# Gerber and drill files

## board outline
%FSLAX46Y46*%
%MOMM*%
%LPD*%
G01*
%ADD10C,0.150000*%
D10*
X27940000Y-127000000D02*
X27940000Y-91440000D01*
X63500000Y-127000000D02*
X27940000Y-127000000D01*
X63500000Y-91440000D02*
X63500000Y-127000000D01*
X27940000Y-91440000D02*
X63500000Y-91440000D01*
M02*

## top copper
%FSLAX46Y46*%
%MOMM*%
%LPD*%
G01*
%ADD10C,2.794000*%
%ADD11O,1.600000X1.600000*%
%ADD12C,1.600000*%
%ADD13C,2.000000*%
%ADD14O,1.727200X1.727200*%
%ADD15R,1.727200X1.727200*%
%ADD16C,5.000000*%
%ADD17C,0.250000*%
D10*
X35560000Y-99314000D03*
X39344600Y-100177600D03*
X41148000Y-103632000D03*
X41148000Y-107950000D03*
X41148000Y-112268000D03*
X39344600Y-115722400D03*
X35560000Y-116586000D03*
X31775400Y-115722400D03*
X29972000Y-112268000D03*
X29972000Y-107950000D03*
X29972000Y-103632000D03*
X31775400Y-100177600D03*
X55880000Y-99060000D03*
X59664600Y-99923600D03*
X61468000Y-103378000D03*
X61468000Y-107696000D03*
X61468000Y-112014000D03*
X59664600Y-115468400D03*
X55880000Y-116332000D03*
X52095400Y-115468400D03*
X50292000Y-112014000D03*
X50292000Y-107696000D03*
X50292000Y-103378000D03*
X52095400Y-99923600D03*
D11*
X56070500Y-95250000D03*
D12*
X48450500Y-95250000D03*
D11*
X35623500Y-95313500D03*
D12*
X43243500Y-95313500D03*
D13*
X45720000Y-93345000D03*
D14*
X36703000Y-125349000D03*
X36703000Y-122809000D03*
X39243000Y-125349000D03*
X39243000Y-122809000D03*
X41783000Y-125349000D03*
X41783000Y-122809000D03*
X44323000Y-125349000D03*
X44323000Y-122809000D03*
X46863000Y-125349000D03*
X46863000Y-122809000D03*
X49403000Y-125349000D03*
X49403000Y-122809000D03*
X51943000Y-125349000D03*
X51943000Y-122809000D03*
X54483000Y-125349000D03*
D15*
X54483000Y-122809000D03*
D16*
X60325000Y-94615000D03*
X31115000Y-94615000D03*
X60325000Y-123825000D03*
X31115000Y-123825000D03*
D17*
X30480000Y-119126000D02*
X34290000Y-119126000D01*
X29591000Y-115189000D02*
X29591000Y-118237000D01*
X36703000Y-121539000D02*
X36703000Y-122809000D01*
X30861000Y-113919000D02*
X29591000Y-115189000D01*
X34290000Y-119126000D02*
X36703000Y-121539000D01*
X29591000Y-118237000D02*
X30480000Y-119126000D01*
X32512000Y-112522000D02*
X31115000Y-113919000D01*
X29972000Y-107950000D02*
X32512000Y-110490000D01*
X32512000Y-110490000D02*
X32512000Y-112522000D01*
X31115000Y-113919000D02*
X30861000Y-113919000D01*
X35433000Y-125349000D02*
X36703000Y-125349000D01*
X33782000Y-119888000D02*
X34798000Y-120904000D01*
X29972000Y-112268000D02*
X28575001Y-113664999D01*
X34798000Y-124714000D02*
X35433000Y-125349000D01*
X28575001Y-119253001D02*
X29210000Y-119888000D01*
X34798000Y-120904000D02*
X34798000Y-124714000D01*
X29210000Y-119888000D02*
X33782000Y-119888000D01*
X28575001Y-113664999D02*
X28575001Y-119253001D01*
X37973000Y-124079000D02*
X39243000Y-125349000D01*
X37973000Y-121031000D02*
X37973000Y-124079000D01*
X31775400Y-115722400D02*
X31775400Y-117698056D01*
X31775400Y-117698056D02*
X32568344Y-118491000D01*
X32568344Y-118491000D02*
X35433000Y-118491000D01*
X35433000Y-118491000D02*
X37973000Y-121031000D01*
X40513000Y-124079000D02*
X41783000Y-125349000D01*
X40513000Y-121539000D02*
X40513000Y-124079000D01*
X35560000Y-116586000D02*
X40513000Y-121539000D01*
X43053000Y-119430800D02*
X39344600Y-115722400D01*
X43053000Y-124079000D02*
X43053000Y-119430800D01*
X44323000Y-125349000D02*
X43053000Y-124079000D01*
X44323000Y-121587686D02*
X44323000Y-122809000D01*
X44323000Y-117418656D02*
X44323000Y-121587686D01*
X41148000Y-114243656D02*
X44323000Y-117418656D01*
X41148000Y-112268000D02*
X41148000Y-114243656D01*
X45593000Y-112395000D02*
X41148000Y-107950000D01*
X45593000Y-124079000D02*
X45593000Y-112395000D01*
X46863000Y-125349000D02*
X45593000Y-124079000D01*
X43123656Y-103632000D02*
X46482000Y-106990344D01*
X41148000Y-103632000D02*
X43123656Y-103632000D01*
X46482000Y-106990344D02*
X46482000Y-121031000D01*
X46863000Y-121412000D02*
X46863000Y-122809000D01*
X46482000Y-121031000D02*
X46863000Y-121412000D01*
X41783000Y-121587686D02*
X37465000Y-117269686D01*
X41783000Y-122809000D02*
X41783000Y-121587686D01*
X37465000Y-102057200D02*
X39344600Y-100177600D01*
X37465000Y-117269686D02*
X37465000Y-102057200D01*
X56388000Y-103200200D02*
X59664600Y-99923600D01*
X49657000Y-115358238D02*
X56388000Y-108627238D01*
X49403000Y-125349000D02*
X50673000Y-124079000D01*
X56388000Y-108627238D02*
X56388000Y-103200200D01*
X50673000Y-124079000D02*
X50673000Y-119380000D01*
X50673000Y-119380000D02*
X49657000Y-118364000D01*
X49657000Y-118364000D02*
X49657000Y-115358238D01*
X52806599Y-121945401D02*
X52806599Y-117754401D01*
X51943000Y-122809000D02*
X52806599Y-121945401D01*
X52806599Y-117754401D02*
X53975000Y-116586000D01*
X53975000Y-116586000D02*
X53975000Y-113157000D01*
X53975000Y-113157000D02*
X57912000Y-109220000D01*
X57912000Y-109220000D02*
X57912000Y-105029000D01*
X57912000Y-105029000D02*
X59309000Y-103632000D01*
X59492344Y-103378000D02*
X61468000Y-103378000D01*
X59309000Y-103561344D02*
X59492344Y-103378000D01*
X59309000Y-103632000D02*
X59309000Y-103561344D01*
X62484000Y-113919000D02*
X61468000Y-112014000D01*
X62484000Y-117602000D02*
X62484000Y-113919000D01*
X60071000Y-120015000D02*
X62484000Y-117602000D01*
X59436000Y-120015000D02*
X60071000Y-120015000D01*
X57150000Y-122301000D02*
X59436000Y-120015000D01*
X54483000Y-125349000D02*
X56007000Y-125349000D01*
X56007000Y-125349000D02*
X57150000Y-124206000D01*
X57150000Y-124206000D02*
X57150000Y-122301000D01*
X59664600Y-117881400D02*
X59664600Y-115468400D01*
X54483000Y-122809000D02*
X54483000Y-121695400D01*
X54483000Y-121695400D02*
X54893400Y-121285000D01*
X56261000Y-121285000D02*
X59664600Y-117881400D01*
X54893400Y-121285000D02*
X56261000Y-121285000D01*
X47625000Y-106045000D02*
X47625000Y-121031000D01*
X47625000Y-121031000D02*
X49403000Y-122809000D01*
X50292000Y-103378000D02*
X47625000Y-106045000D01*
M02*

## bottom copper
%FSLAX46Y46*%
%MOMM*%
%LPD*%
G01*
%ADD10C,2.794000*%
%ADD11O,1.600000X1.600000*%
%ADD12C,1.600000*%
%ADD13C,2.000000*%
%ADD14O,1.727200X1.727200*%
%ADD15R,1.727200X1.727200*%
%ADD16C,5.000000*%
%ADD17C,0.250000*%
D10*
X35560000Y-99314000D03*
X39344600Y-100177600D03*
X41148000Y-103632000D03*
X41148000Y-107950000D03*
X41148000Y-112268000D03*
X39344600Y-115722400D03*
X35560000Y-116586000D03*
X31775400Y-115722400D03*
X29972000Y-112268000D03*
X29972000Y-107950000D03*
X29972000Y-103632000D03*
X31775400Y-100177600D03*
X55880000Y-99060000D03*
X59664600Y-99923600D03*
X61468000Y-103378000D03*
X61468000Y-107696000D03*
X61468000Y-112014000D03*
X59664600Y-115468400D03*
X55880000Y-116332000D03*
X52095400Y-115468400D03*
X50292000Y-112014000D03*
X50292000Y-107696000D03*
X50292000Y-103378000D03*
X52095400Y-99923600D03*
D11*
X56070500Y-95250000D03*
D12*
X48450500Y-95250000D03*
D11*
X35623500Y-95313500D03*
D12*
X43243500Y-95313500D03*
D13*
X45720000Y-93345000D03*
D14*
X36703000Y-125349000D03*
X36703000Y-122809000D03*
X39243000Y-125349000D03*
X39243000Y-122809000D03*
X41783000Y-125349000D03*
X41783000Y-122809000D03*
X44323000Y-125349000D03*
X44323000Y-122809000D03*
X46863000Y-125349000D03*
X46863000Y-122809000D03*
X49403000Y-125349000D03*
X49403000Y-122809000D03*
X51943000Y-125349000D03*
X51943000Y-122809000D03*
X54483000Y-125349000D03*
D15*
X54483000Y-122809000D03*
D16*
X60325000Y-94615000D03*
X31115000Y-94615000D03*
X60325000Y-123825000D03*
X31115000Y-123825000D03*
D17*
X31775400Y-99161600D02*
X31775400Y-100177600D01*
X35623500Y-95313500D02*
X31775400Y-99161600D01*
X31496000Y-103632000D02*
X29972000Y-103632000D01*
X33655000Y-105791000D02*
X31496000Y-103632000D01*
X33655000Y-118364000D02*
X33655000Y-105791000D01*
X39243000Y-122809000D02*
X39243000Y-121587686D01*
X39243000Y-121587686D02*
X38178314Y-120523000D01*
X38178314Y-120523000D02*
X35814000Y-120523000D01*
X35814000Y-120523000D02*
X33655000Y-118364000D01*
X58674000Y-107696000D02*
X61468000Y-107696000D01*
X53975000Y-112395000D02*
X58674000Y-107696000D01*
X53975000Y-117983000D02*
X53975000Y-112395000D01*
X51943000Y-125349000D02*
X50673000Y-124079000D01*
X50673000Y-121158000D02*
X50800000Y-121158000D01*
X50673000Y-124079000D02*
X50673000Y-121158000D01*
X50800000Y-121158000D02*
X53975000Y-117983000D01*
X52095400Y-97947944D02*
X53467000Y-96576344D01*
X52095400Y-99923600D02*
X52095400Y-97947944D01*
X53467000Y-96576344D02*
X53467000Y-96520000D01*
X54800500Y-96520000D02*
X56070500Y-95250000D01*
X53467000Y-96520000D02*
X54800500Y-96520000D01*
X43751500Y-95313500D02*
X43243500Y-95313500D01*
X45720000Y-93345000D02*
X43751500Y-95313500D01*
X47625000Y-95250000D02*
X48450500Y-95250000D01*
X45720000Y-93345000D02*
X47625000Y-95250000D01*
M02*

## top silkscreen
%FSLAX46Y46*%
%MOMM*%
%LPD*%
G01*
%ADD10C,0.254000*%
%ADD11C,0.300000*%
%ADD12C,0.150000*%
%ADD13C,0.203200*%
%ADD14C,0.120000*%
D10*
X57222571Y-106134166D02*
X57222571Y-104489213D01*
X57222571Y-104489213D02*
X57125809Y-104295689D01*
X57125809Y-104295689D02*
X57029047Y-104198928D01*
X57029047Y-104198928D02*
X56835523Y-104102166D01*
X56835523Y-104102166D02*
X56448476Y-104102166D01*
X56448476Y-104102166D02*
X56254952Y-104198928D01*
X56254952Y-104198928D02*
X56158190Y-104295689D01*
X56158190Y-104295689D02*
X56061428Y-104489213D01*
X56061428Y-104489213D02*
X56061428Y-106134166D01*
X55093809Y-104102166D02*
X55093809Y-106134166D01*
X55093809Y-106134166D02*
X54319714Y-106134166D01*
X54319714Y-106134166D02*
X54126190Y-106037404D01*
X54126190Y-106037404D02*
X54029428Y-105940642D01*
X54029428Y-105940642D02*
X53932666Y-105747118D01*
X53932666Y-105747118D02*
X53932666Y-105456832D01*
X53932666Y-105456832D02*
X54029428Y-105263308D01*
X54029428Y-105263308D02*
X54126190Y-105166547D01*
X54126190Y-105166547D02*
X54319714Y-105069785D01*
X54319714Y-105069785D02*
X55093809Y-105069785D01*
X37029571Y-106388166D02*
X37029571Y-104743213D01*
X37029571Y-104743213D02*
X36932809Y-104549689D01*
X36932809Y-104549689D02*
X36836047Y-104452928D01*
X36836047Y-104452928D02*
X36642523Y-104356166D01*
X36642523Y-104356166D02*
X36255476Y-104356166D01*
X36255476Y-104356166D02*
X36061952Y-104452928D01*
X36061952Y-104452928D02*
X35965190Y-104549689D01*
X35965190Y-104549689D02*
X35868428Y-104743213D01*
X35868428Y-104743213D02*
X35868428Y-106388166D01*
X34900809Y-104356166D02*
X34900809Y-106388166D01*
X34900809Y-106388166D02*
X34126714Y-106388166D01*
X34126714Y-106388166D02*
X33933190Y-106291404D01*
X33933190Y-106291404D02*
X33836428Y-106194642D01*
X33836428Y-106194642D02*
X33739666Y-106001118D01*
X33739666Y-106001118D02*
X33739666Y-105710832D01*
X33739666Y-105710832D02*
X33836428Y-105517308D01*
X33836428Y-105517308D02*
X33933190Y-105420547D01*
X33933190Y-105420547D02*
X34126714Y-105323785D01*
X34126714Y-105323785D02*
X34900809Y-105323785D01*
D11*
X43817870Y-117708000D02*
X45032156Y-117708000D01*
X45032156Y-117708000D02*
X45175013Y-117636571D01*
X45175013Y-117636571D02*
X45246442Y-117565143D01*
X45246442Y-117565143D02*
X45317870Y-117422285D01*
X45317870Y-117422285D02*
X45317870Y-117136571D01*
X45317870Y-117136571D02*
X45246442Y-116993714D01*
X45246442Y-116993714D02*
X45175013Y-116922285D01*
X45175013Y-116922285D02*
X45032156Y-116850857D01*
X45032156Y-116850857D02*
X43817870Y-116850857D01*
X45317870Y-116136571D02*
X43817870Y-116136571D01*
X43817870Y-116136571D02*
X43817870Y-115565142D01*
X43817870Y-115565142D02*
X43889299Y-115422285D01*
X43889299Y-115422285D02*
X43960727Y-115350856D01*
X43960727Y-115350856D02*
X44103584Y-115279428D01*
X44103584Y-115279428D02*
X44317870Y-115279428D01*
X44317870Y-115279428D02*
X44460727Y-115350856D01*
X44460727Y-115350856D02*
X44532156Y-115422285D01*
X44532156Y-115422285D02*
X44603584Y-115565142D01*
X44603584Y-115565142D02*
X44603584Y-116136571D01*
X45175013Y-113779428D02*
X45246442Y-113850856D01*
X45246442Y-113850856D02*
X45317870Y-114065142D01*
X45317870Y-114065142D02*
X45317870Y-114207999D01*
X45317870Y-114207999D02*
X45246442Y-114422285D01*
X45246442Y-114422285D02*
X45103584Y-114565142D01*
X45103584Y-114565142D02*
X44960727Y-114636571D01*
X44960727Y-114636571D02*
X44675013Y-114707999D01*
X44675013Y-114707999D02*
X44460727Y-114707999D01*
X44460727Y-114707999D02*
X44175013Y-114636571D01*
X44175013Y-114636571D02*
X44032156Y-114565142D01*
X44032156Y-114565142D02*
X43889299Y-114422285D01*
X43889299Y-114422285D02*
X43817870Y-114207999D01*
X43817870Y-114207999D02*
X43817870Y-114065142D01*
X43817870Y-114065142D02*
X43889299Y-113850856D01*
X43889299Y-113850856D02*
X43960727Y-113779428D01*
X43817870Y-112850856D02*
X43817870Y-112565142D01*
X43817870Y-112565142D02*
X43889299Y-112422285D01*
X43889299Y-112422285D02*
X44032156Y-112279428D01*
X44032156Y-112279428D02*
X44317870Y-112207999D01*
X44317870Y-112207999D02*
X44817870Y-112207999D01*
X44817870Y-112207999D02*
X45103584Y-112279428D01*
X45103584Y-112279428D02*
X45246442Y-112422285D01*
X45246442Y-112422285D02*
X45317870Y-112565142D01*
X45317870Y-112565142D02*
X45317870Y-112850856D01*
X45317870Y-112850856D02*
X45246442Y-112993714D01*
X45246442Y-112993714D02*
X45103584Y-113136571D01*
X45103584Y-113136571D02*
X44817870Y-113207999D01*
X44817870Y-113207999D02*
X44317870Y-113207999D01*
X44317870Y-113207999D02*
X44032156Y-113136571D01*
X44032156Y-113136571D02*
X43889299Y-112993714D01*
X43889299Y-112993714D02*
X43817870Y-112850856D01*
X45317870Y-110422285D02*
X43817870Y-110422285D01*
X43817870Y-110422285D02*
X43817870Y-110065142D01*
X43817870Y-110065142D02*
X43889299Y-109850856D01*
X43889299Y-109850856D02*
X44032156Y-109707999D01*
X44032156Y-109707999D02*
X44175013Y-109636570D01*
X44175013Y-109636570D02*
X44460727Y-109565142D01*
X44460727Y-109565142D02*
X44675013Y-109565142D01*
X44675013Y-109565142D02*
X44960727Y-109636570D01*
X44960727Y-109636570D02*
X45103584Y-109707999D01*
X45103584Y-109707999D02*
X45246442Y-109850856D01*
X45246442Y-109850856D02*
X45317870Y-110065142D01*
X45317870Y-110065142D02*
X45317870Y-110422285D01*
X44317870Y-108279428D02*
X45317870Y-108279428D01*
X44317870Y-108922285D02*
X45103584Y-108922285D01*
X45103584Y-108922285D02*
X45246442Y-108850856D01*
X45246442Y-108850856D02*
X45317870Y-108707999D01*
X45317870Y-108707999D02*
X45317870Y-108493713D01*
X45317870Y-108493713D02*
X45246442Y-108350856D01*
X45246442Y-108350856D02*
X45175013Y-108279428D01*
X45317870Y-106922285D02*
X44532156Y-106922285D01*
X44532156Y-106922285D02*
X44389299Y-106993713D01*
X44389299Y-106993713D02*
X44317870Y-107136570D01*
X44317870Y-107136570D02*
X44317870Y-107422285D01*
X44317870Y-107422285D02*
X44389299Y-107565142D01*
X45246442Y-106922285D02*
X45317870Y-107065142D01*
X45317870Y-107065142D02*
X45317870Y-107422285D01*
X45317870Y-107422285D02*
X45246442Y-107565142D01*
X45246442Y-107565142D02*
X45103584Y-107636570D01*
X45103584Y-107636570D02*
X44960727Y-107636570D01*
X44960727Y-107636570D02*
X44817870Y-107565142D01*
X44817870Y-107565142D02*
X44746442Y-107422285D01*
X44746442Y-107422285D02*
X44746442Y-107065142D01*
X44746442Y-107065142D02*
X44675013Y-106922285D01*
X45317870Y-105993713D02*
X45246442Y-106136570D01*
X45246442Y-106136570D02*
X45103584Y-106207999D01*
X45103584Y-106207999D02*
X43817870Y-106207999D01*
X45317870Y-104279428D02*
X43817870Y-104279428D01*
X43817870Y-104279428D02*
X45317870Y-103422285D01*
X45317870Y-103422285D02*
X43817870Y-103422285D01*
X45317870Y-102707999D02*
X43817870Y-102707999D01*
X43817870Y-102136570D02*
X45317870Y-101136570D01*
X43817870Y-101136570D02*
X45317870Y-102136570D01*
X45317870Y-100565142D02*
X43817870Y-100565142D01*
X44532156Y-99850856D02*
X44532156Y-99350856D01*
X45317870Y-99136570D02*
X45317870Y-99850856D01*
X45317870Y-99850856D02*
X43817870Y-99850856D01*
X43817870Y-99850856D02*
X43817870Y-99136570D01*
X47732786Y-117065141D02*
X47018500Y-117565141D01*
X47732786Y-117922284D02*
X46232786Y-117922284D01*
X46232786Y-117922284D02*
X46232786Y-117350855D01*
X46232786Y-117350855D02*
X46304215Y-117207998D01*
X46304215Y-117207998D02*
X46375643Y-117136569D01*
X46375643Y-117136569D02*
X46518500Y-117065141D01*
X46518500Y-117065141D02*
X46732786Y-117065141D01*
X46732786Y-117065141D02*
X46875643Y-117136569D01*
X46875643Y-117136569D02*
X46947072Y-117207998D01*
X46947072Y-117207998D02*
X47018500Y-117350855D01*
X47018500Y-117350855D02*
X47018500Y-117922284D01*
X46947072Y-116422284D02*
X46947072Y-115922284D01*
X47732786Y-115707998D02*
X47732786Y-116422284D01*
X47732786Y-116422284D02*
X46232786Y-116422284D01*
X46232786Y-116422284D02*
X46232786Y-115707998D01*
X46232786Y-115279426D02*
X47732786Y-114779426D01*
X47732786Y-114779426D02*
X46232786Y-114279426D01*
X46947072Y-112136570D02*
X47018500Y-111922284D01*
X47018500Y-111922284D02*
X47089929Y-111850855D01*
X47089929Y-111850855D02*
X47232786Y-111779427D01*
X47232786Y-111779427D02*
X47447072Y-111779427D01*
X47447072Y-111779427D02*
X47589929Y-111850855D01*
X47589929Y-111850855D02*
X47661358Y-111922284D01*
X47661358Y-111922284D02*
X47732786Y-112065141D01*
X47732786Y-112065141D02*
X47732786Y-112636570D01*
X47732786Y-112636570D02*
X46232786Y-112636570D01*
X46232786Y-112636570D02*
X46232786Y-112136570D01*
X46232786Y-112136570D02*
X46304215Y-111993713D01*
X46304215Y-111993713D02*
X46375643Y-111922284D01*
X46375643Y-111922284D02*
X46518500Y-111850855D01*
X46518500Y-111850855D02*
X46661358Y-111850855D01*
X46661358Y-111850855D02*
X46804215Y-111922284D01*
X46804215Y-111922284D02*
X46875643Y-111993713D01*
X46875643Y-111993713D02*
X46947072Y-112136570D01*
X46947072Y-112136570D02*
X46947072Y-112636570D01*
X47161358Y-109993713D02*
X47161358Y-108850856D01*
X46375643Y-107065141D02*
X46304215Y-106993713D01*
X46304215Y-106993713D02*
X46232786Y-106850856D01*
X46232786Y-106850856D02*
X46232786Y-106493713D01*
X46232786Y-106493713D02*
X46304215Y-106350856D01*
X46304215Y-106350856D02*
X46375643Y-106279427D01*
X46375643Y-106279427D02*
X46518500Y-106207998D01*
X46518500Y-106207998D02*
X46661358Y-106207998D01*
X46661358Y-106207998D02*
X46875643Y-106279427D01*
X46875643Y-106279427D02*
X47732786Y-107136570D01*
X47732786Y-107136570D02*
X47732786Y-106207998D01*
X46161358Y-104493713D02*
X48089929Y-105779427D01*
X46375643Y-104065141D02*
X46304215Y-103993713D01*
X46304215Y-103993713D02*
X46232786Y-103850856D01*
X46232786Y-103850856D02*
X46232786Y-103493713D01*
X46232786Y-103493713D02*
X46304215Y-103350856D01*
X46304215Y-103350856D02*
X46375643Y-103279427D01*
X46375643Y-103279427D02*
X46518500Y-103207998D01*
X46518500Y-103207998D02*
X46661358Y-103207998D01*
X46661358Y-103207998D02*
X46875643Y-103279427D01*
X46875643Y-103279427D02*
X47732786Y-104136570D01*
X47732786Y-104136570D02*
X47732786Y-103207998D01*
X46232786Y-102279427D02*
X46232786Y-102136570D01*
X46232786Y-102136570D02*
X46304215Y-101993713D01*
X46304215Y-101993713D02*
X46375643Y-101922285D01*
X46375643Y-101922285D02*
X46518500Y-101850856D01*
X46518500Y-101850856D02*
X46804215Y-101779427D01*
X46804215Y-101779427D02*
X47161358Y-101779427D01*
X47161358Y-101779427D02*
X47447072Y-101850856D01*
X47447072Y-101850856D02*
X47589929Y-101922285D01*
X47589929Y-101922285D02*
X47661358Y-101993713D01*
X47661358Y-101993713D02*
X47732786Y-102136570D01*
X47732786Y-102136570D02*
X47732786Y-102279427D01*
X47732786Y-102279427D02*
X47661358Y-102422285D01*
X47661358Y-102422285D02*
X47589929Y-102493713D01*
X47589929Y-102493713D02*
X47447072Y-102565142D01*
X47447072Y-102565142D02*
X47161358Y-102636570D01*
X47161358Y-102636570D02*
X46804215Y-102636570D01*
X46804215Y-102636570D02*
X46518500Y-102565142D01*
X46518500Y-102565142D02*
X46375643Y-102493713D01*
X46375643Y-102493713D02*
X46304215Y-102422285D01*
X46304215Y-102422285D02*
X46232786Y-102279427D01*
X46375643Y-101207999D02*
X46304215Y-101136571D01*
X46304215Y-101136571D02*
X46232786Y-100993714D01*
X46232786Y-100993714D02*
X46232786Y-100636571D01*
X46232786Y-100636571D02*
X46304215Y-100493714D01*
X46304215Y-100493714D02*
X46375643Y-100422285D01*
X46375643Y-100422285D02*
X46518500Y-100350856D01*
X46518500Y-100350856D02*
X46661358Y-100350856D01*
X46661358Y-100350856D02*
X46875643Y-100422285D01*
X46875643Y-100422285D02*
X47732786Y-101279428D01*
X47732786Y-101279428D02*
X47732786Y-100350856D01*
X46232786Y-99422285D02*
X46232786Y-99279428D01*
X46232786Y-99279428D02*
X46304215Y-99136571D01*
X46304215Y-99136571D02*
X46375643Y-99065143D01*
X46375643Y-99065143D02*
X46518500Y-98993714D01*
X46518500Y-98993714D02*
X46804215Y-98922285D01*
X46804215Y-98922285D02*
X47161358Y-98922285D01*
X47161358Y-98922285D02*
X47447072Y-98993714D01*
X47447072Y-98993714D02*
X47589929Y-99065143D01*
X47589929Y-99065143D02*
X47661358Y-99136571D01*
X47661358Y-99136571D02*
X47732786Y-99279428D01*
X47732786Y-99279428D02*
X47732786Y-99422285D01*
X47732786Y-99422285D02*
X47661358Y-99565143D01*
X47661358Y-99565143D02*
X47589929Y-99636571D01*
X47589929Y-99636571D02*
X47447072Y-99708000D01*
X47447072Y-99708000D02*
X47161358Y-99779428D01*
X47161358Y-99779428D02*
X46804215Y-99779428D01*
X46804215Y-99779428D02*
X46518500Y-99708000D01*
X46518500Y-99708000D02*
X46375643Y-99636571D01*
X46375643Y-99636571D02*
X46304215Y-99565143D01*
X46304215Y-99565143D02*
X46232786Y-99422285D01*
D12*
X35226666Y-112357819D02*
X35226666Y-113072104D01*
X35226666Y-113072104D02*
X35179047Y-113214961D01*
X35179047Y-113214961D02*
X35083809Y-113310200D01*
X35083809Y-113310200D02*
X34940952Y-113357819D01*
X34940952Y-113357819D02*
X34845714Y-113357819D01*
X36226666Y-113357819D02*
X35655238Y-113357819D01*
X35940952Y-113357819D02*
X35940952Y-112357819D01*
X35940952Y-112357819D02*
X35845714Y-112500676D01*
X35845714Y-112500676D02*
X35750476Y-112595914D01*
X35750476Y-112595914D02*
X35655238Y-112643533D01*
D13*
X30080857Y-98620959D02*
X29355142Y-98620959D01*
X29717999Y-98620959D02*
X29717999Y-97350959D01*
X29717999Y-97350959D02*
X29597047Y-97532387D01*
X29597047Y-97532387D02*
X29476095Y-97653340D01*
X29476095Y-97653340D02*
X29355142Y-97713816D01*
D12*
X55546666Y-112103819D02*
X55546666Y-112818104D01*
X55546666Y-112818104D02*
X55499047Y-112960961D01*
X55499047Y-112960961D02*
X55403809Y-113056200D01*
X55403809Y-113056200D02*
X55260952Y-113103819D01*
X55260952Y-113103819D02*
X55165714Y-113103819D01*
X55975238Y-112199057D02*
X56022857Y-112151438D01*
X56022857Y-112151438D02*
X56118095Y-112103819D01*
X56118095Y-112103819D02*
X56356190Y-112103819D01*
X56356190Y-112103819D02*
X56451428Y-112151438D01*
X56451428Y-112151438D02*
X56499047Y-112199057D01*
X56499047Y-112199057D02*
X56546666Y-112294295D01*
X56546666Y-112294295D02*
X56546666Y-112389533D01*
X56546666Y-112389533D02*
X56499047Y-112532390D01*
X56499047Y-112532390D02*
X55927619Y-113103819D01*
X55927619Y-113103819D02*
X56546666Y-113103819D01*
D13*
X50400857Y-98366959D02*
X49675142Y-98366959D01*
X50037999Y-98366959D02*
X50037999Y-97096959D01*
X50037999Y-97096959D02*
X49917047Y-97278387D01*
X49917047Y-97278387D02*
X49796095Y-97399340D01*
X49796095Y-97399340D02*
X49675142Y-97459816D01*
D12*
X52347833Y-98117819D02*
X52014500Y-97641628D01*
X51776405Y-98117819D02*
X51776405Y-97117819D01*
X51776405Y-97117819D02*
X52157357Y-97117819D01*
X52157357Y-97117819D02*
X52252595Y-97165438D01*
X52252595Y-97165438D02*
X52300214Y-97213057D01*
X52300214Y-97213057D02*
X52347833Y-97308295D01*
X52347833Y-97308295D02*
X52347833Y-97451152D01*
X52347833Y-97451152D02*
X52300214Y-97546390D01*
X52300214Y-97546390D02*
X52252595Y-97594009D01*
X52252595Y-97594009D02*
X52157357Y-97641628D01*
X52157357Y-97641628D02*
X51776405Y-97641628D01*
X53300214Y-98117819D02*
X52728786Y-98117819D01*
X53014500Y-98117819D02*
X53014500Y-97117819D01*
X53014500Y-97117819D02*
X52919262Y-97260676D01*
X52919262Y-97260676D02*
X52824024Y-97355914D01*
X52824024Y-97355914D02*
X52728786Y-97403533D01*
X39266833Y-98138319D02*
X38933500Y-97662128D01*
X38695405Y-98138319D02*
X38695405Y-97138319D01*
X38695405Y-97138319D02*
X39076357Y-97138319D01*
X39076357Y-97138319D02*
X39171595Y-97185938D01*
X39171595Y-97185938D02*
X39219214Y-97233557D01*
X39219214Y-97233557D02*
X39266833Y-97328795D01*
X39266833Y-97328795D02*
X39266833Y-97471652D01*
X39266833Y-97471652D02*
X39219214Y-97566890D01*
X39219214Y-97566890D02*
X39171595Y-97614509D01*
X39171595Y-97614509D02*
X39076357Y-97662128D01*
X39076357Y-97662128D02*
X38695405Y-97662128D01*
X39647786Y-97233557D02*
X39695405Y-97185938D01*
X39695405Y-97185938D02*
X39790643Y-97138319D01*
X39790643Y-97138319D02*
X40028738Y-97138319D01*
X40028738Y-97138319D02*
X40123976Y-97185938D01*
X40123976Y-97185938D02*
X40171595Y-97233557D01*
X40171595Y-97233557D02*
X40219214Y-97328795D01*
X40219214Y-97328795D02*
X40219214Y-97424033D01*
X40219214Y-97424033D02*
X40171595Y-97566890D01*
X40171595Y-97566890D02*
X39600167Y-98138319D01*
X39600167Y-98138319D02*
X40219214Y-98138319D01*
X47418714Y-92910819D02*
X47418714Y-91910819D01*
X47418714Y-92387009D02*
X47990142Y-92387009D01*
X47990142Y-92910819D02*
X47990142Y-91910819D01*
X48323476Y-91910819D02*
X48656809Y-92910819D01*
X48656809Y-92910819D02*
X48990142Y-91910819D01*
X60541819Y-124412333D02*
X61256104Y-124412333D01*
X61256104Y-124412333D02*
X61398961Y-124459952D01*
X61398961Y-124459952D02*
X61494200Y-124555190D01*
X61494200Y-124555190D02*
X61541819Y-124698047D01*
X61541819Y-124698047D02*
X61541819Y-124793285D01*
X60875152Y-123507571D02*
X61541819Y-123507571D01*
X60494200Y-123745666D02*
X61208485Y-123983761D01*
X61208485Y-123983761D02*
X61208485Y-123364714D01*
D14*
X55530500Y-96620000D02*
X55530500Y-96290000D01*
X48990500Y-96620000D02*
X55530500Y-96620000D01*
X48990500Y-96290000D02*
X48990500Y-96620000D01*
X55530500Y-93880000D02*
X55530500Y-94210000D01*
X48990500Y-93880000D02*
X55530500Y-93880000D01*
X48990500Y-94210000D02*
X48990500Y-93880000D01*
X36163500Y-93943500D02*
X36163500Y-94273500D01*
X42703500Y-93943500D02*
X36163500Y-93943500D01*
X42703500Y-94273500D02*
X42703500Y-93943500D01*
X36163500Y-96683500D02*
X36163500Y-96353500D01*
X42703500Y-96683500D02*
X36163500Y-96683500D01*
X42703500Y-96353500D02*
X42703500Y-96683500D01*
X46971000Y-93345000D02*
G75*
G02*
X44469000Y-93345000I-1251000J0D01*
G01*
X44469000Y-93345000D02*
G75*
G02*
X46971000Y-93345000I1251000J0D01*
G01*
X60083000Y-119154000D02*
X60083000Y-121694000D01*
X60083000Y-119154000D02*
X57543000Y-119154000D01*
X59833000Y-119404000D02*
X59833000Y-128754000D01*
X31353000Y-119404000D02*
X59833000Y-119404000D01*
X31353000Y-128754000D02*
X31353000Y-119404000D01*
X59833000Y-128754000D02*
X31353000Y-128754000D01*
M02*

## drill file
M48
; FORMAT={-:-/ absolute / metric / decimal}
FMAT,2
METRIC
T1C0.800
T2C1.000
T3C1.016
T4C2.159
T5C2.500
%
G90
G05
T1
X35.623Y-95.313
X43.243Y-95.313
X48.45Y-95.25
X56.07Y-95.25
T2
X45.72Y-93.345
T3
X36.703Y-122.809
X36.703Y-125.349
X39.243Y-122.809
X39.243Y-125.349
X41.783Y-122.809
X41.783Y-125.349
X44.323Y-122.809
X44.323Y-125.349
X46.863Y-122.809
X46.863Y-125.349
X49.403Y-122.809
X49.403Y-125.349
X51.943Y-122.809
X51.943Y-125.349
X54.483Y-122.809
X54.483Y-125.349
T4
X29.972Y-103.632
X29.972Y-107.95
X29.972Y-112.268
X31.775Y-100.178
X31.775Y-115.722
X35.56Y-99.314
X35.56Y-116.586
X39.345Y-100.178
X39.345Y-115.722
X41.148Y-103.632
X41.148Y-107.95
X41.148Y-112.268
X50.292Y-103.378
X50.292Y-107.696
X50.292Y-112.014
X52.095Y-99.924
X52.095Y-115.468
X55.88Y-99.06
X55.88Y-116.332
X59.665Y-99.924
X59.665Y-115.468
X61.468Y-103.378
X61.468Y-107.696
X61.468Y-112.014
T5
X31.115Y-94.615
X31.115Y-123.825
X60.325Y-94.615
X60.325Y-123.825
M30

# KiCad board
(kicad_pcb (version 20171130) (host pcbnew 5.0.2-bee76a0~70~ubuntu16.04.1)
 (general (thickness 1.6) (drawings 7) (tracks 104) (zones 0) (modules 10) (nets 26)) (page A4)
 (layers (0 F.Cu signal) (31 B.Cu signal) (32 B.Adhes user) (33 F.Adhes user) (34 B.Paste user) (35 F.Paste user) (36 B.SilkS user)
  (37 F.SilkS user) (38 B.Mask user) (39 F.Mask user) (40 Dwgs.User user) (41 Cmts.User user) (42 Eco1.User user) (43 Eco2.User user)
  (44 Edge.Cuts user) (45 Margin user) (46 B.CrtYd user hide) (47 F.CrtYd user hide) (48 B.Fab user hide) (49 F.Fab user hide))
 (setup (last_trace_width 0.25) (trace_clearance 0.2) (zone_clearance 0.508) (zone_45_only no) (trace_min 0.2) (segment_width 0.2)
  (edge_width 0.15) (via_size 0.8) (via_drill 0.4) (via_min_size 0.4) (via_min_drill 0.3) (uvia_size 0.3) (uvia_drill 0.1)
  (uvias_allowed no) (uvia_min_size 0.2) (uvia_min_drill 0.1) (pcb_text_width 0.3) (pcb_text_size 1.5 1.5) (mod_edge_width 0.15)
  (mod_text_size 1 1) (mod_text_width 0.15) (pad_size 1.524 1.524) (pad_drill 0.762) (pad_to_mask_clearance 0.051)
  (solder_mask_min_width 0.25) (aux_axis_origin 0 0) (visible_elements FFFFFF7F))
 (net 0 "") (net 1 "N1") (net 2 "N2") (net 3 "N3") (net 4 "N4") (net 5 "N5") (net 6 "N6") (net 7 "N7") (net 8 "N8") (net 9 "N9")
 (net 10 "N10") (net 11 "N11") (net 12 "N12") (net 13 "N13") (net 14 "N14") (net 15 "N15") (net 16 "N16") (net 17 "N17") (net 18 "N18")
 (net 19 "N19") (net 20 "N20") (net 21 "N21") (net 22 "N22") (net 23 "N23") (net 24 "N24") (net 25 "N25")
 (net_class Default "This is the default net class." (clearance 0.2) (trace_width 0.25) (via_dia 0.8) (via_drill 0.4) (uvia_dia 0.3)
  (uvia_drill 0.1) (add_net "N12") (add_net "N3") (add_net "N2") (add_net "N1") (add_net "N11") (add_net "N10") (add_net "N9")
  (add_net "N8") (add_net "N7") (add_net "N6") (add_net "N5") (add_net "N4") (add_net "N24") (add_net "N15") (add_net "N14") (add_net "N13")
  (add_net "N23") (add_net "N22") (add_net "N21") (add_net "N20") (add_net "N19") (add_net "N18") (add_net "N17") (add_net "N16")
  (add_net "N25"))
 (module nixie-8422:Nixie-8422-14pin (layer F.Cu) (at 35.56 107.95)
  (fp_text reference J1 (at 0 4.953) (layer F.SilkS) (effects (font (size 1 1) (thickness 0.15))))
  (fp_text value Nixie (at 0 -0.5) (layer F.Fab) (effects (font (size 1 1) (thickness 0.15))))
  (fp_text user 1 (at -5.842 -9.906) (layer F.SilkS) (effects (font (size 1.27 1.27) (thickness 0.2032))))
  (pad 12 thru_hole circle (at 0 -8.636) (size 2.794 2.794) (drill 2.159) (layers *.Cu *.Mask) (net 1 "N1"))
  (pad 11 thru_hole circle (at 3.7846 -7.7724) (size 2.794 2.794) (drill 2.159) (layers *.Cu *.Mask) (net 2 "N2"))
  (pad 10 thru_hole circle (at 5.588 -4.318) (size 2.794 2.794) (drill 2.159) (layers *.Cu *.Mask) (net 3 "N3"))
  (pad 9 thru_hole circle (at 5.588 0) (size 2.794 2.794) (drill 2.159) (layers *.Cu *.Mask) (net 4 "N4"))
  (pad 8 thru_hole circle (at 5.588 4.318) (size 2.794 2.794) (drill 2.159) (layers *.Cu *.Mask) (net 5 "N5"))
  (pad 7 thru_hole circle (at 3.7846 7.7724) (size 2.794 2.794) (drill 2.159) (layers *.Cu *.Mask) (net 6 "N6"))
  (pad 6 thru_hole circle (at 0 8.636) (size 2.794 2.794) (drill 2.159) (layers *.Cu *.Mask) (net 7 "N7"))
  (pad 5 thru_hole circle (at -3.7846 7.7724) (size 2.794 2.794) (drill 2.159) (layers *.Cu *.Mask) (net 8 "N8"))
  (pad 4 thru_hole circle (at -5.588 4.318) (size 2.794 2.794) (drill 2.159) (layers *.Cu *.Mask) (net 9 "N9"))
  (pad 3 thru_hole circle (at -5.588 0) (size 2.794 2.794) (drill 2.159) (layers *.Cu *.Mask) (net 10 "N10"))
  (pad 2 thru_hole circle (at -5.588 -4.318) (size 2.794 2.794) (drill 2.159) (layers *.Cu *.Mask) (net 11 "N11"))
  (pad 1 thru_hole circle (at -3.7846 -7.7724) (size 2.794 2.794) (drill 2.159) (layers *.Cu *.Mask) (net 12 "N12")))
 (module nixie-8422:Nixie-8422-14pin (layer F.Cu) (at 55.88 107.696)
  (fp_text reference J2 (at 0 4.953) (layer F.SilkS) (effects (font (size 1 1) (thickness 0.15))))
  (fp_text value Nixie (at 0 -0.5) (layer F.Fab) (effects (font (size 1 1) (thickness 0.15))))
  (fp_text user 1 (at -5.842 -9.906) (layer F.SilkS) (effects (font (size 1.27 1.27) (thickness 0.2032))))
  (pad 12 thru_hole circle (at 0 -8.636) (size 2.794 2.794) (drill 2.159) (layers *.Cu *.Mask) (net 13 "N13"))
  (pad 11 thru_hole circle (at 3.7846 -7.7724) (size 2.794 2.794) (drill 2.159) (layers *.Cu *.Mask) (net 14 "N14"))
  (pad 10 thru_hole circle (at 5.588 -4.318) (size 2.794 2.794) (drill 2.159) (layers *.Cu *.Mask) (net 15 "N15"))
  (pad 9 thru_hole circle (at 5.588 0) (size 2.794 2.794) (drill 2.159) (layers *.Cu *.Mask) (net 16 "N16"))
  (pad 8 thru_hole circle (at 5.588 4.318) (size 2.794 2.794) (drill 2.159) (layers *.Cu *.Mask) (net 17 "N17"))
  (pad 7 thru_hole circle (at 3.7846 7.7724) (size 2.794 2.794) (drill 2.159) (layers *.Cu *.Mask) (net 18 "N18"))
  (pad 6 thru_hole circle (at 0 8.636) (size 2.794 2.794) (drill 2.159) (layers *.Cu *.Mask) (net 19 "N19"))
  (pad 5 thru_hole circle (at -3.7846 7.7724) (size 2.794 2.794) (drill 2.159) (layers *.Cu *.Mask) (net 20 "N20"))
  (pad 4 thru_hole circle (at -5.588 4.318) (size 2.794 2.794) (drill 2.159) (layers *.Cu *.Mask) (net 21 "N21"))
  (pad 3 thru_hole circle (at -5.588 0) (size 2.794 2.794) (drill 2.159) (layers *.Cu *.Mask) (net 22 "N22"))
  (pad 2 thru_hole circle (at -5.588 -4.318) (size 2.794 2.794) (drill 2.159) (layers *.Cu *.Mask) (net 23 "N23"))
  (pad 1 thru_hole circle (at -3.7846 -7.7724) (size 2.794 2.794) (drill 2.159) (layers *.Cu *.Mask) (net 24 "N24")))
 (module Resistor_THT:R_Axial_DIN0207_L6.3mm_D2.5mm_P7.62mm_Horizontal (layer F.Cu) (at 48.4505 95.25)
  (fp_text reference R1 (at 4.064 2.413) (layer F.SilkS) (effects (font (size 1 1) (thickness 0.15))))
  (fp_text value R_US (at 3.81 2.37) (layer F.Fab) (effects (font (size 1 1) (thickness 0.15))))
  (fp_line (start 7.08 1.37) (end 7.08 1.04) (layer F.SilkS) (width 0.12))
  (fp_line (start 0.54 1.37) (end 7.08 1.37) (layer F.SilkS) (width 0.12))
  (fp_line (start 0.54 1.04) (end 0.54 1.37) (layer F.SilkS) (width 0.12))
  (fp_line (start 7.08 -1.37) (end 7.08 -1.04) (layer F.SilkS) (width 0.12))
  (fp_line (start 0.54 -1.37) (end 7.08 -1.37) (layer F.SilkS) (width 0.12))
  (fp_line (start 0.54 -1.04) (end 0.54 -1.37) (layer F.SilkS) (width 0.12))
  (pad 2 thru_hole oval (at 7.62 0) (size 1.6 1.6) (drill 0.8) (layers *.Cu *.Mask) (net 24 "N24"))
  (pad 1 thru_hole circle (at 0 0) (size 1.6 1.6) (drill 0.8) (layers *.Cu *.Mask) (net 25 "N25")))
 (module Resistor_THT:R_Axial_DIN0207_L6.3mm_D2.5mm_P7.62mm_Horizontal (layer F.Cu) (at 43.2435 95.3135 180)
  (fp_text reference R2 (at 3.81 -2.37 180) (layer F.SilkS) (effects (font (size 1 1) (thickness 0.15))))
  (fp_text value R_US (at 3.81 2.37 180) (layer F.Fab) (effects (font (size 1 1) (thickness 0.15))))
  (fp_line (start 7.08 1.37) (end 7.08 1.04) (layer F.SilkS) (width 0.12))
  (fp_line (start 0.54 1.37) (end 7.08 1.37) (layer F.SilkS) (width 0.12))
  (fp_line (start 0.54 1.04) (end 0.54 1.37) (layer F.SilkS) (width 0.12))
  (fp_line (start 7.08 -1.37) (end 7.08 -1.04) (layer F.SilkS) (width 0.12))
  (fp_line (start 0.54 -1.37) (end 7.08 -1.37) (layer F.SilkS) (width 0.12))
  (fp_line (start 0.54 -1.04) (end 0.54 -1.37) (layer F.SilkS) (width 0.12))
  (pad 2 thru_hole oval (at 7.62 0 180) (size 1.6 1.6) (drill 0.8) (layers *.Cu *.Mask) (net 12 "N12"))
  (pad 1 thru_hole circle (at 0 0 180) (size 1.6 1.6) (drill 0.8) (layers *.Cu *.Mask) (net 25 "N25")))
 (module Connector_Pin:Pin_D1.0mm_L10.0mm (layer F.Cu) (at 45.72 93.345)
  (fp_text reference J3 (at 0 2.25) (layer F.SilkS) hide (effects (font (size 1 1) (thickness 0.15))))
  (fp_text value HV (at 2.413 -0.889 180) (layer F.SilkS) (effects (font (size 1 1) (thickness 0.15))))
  (fp_circle (center 0 0) (end 1.25 0.05) (layer F.SilkS) (width 0.12))
  (pad 1 thru_hole circle (at 0 0) (size 2 2) (drill 1) (layers *.Cu *.Mask) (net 25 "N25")))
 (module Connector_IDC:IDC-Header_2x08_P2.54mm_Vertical (layer F.Cu) (at 54.483 122.809 270)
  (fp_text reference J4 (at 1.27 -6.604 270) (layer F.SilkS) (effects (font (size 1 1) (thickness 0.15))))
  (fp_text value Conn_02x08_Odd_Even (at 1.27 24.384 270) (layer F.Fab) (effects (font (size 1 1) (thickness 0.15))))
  (fp_line (start -3.655 -5.6) (end -1.115 -5.6) (layer F.SilkS) (width 0.12))
  (fp_line (start -3.655 -5.6) (end -3.655 -3.06) (layer F.SilkS) (width 0.12))
  (fp_line (start -3.405 -5.35) (end 5.945 -5.35) (layer F.SilkS) (width 0.12))
  (fp_line (start -3.405 23.13) (end -3.405 -5.35) (layer F.SilkS) (width 0.12))
  (fp_line (start 5.945 23.13) (end -3.405 23.13) (layer F.SilkS) (width 0.12))
  (fp_line (start 5.945 -5.35) (end 5.945 23.13) (layer F.SilkS) (width 0.12))
  (pad 16 thru_hole oval (at 2.54 17.78 270) (size 1.7272 1.7272) (drill 1.016) (layers *.Cu *.Mask) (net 9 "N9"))
  (pad 15 thru_hole oval (at 0 17.78 270) (size 1.7272 1.7272) (drill 1.016) (layers *.Cu *.Mask) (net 10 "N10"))
  (pad 14 thru_hole oval (at 2.54 15.24 270) (size 1.7272 1.7272) (drill 1.016) (layers *.Cu *.Mask) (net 8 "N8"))
  (pad 13 thru_hole oval (at 0 15.24 270) (size 1.7272 1.7272) (drill 1.016) (layers *.Cu *.Mask) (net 11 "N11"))
  (pad 12 thru_hole oval (at 2.54 12.7 270) (size 1.7272 1.7272) (drill 1.016) (layers *.Cu *.Mask) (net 7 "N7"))
  (pad 11 thru_hole oval (at 0 12.7 270) (size 1.7272 1.7272) (drill 1.016) (layers *.Cu *.Mask) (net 2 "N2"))
  (pad 10 thru_hole oval (at 2.54 10.16 270) (size 1.7272 1.7272) (drill 1.016) (layers *.Cu *.Mask) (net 6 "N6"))
  (pad 9 thru_hole oval (at 0 10.16 270) (size 1.7272 1.7272) (drill 1.016) (layers *.Cu *.Mask) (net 5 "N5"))
  (pad 8 thru_hole oval (at 2.54 7.62 270) (size 1.7272 1.7272) (drill 1.016) (layers *.Cu *.Mask) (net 4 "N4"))
  (pad 7 thru_hole oval (at 0 7.62 270) (size 1.7272 1.7272) (drill 1.016) (layers *.Cu *.Mask) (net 3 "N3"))
  (pad 6 thru_hole oval (at 2.54 5.08 270) (size 1.7272 1.7272) (drill 1.016) (layers *.Cu *.Mask) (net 14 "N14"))
  (pad 5 thru_hole oval (at 0 5.08 270) (size 1.7272 1.7272) (drill 1.016) (layers *.Cu *.Mask) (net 23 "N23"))
  (pad 4 thru_hole oval (at 2.54 2.54 270) (size 1.7272 1.7272) (drill 1.016) (layers *.Cu *.Mask) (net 16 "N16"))
  (pad 3 thru_hole oval (at 0 2.54 270) (size 1.7272 1.7272) (drill 1.016) (layers *.Cu *.Mask) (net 15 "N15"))
  (pad 2 thru_hole oval (at 2.54 0 270) (size 1.7272 1.7272) (drill 1.016) (layers *.Cu *.Mask) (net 17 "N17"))
  (pad 1 thru_hole rect (at 0 0 270) (size 1.7272 1.7272) (drill 1.016) (layers *.Cu *.Mask) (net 18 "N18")))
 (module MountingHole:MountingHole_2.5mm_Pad (layer F.Cu) (at 60.325 94.615)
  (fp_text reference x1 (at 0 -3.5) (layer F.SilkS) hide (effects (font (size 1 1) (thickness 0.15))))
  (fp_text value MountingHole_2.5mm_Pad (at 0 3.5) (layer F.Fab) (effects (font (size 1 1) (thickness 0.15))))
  (pad 1 thru_hole circle (at 0 0) (size 5 5) (drill 2.5) (layers *.Cu *.Mask)))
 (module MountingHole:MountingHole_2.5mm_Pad (layer F.Cu) (at 31.115 94.615)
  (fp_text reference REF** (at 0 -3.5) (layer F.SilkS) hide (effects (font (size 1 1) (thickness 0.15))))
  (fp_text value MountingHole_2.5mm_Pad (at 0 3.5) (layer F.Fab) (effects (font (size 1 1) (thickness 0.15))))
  (pad 1 thru_hole circle (at 0 0) (size 5 5) (drill 2.5) (layers *.Cu *.Mask)))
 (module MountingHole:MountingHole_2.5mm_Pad (layer F.Cu) (at 60.325 123.825)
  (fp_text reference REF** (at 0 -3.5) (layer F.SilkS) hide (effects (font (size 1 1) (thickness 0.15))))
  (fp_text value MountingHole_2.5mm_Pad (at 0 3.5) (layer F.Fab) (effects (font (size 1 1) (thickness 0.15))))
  (pad 1 thru_hole circle (at 0 0) (size 5 5) (drill 2.5) (layers *.Cu *.Mask)))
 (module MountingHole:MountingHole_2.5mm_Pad (layer F.Cu) (at 31.115 123.825)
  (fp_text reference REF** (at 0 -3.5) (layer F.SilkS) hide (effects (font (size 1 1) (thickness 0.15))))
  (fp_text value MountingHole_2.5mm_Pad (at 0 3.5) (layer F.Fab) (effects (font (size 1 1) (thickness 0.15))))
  (pad 1 thru_hole circle (at 0 0) (size 5 5) (drill 2.5) (layers *.Cu *.Mask)))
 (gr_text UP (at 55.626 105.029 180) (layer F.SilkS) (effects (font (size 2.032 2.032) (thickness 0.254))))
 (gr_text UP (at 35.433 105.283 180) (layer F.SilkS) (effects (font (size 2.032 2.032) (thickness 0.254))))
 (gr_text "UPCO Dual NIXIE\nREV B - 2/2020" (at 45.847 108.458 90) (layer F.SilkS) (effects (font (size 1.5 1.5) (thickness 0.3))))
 (gr_line (start 27.94 127) (end 27.94 91.44) (layer Edge.Cuts) (width 0.15))
 (gr_line (start 63.5 127) (end 27.94 127) (layer Edge.Cuts) (width 0.15))
 (gr_line (start 63.5 91.44) (end 63.5 127) (layer Edge.Cuts) (width 0.15))
 (gr_line (start 27.94 91.44) (end 63.5 91.44) (layer Edge.Cuts) (width 0.15))
 (segment (start 31.7754 99.1616) (end 31.7754 100.1776) (width 0.25) (layer B.Cu) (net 12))
 (segment (start 35.6235 95.3135) (end 31.7754 99.1616) (width 0.25) (layer B.Cu) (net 12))
 (segment (start 31.496 103.632) (end 29.972 103.632) (width 0.25) (layer B.Cu) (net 11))
 (segment (start 33.655 105.791) (end 31.496 103.632) (width 0.25) (layer B.Cu) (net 11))
 (segment (start 33.655 118.364) (end 33.655 105.791) (width 0.25) (layer B.Cu) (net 11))
 (segment (start 39.243 122.809) (end 39.243 121.587686) (width 0.25) (layer B.Cu) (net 11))
 (segment (start 39.243 121.587686) (end 38.178314 120.523) (width 0.25) (layer B.Cu) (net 11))
 (segment (start 38.178314 120.523) (end 35.814 120.523) (width 0.25) (layer B.Cu) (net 11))
 (segment (start 35.814 120.523) (end 33.655 118.364) (width 0.25) (layer B.Cu) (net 11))
 (segment (start 30.48 119.126) (end 34.29 119.126) (width 0.25) (layer F.Cu) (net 10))
 (segment (start 29.591 115.189) (end 29.591 118.237) (width 0.25) (layer F.Cu) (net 10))
 (segment (start 36.703 121.539) (end 36.703 122.809) (width 0.25) (layer F.Cu) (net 10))
 (segment (start 30.861 113.919) (end 29.591 115.189) (width 0.25) (layer F.Cu) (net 10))
 (segment (start 34.29 119.126) (end 36.703 121.539) (width 0.25) (layer F.Cu) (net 10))
 (segment (start 29.591 118.237) (end 30.48 119.126) (width 0.25) (layer F.Cu) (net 10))
 (segment (start 32.512 112.522) (end 31.115 113.919) (width 0.25) (layer F.Cu) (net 10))
 (segment (start 29.972 107.95) (end 32.512 110.49) (width 0.25) (layer F.Cu) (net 10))
 (segment (start 32.512 110.49) (end 32.512 112.522) (width 0.25) (layer F.Cu) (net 10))
 (segment (start 31.115 113.919) (end 30.861 113.919) (width 0.25) (layer F.Cu) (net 10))
 (segment (start 35.433 125.349) (end 36.703 125.349) (width 0.25) (layer F.Cu) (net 9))
 (segment (start 33.782 119.888) (end 34.798 120.904) (width 0.25) (layer F.Cu) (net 9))
 (segment (start 29.972 112.268) (end 28.575001 113.664999) (width 0.25) (layer F.Cu) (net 9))
 (segment (start 34.798 124.714) (end 35.433 125.349) (width 0.25) (layer F.Cu) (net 9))
 (segment (start 28.575001 119.253001) (end 29.21 119.888) (width 0.25) (layer F.Cu) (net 9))
 (segment (start 34.798 120.904) (end 34.798 124.714) (width 0.25) (layer F.Cu) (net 9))
 (segment (start 29.21 119.888) (end 33.782 119.888) (width 0.25) (layer F.Cu) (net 9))
 (segment (start 28.575001 113.664999) (end 28.575001 119.253001) (width 0.25) (layer F.Cu) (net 9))
 (segment (start 37.973 124.079) (end 39.243 125.349) (width 0.25) (layer F.Cu) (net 8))
 (segment (start 37.973 121.031) (end 37.973 124.079) (width 0.25) (layer F.Cu) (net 8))
 (segment (start 31.7754 115.7224) (end 31.7754 117.698056) (width 0.25) (layer F.Cu) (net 8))
 (segment (start 31.7754 117.698056) (end 32.568344 118.491) (width 0.25) (layer F.Cu) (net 8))
 (segment (start 32.568344 118.491) (end 35.433 118.491) (width 0.25) (layer F.Cu) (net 8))
 (segment (start 35.433 118.491) (end 37.973 121.031) (width 0.25) (layer F.Cu) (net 8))
 (segment (start 40.513 124.079) (end 41.783 125.349) (width 0.25) (layer F.Cu) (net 7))
 (segment (start 40.513 121.539) (end 40.513 124.079) (width 0.25) (layer F.Cu) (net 7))
 (segment (start 35.56 116.586) (end 40.513 121.539) (width 0.25) (layer F.Cu) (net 7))
 (segment (start 43.053 119.4308) (end 39.3446 115.7224) (width 0.25) (layer F.Cu) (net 6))
 (segment (start 43.053 124.079) (end 43.053 119.4308) (width 0.25) (layer F.Cu) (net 6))
 (segment (start 44.323 125.349) (end 43.053 124.079) (width 0.25) (layer F.Cu) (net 6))
 (segment (start 44.323 121.587686) (end 44.323 122.809) (width 0.25) (layer F.Cu) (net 5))
 (segment (start 44.323 117.418656) (end 44.323 121.587686) (width 0.25) (layer F.Cu) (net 5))
 (segment (start 41.148 114.243656) (end 44.323 117.418656) (width 0.25) (layer F.Cu) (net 5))
 (segment (start 41.148 112.268) (end 41.148 114.243656) (width 0.25) (layer F.Cu) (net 5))
 (segment (start 45.593 112.395) (end 41.148 107.95) (width 0.25) (layer F.Cu) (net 4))
 (segment (start 45.593 124.079) (end 45.593 112.395) (width 0.25) (layer F.Cu) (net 4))
 (segment (start 46.863 125.349) (end 45.593 124.079) (width 0.25) (layer F.Cu) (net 4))
 (segment (start 43.123656 103.632) (end 46.482 106.990344) (width 0.25) (layer F.Cu) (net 3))
 (segment (start 41.148 103.632) (end 43.123656 103.632) (width 0.25) (layer F.Cu) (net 3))
 (segment (start 46.482 106.990344) (end 46.482 121.031) (width 0.25) (layer F.Cu) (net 3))
 (segment (start 46.863 121.412) (end 46.863 122.809) (width 0.25) (layer F.Cu) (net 3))
 (segment (start 46.482 121.031) (end 46.863 121.412) (width 0.25) (layer F.Cu) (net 3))
 (segment (start 41.783 121.587686) (end 37.465 117.269686) (width 0.25) (layer F.Cu) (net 2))
 (segment (start 41.783 122.809) (end 41.783 121.587686) (width 0.25) (layer F.Cu) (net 2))
 (segment (start 37.465 102.0572) (end 39.3446 100.1776) (width 0.25) (layer F.Cu) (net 2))
 (segment (start 37.465 117.269686) (end 37.465 102.0572) (width 0.25) (layer F.Cu) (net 2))
 (segment (start 56.388 103.2002) (end 59.6646 99.9236) (width 0.25) (layer F.Cu) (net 14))
 (segment (start 49.657 115.358238) (end 56.388 108.627238) (width 0.25) (layer F.Cu) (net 14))
 (segment (start 49.403 125.349) (end 50.673 124.079) (width 0.25) (layer F.Cu) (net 14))
 (segment (start 56.388 108.627238) (end 56.388 103.2002) (width 0.25) (layer F.Cu) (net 14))
 (segment (start 50.673 124.079) (end 50.673 119.38) (width 0.25) (layer F.Cu) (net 14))
 (segment (start 50.673 119.38) (end 49.657 118.364) (width 0.25) (layer F.Cu) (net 14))
 (segment (start 49.657 118.364) (end 49.657 115.358238) (width 0.25) (layer F.Cu) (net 14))
 (segment (start 52.806599 121.945401) (end 52.806599 117.754401) (width 0.25) (layer F.Cu) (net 15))
 (segment (start 51.943 122.809) (end 52.806599 121.945401) (width 0.25) (layer F.Cu) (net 15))
 (segment (start 52.806599 117.754401) (end 53.975 116.586) (width 0.25) (layer F.Cu) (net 15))
 (segment (start 53.975 116.586) (end 53.975 113.157) (width 0.25) (layer F.Cu) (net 15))
 (segment (start 53.975 113.157) (end 57.912 109.22) (width 0.25) (layer F.Cu) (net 15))
 (segment (start 57.912 109.22) (end 57.912 105.029) (width 0.25) (layer F.Cu) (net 15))
 (segment (start 57.912 105.029) (end 59.309 103.632) (width 0.25) (layer F.Cu) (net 15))
 (segment (start 59.492344 103.378) (end 61.468 103.378) (width 0.25) (layer F.Cu) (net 15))
 (segment (start 59.309 103.561344) (end 59.492344 103.378) (width 0.25) (layer F.Cu) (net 15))
 (segment (start 59.309 103.632) (end 59.309 103.561344) (width 0.25) (layer F.Cu) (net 15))
 (segment (start 58.674 107.696) (end 61.468 107.696) (width 0.25) (layer B.Cu) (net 16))
 (segment (start 53.975 112.395) (end 58.674 107.696) (width 0.25) (layer B.Cu) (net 16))
 (segment (start 53.975 117.983) (end 53.975 112.395) (width 0.25) (layer B.Cu) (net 16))
 (segment (start 51.943 125.349) (end 50.673 124.079) (width 0.25) (layer B.Cu) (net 16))
 (segment (start 50.673 121.158) (end 50.8 121.158) (width 0.25) (layer B.Cu) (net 16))
 (segment (start 50.673 124.079) (end 50.673 121.158) (width 0.25) (layer B.Cu) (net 16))
 (segment (start 50.8 121.158) (end 53.975 117.983) (width 0.25) (layer B.Cu) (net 16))
 (segment (start 62.484 113.919) (end 61.468 112.014) (width 0.25) (layer F.Cu) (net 17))
 (segment (start 62.484 117.602) (end 62.484 113.919) (width 0.25) (layer F.Cu) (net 17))
 (segment (start 60.071 120.015) (end 62.484 117.602) (width 0.25) (layer F.Cu) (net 17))
 (segment (start 59.436 120.015) (end 60.071 120.015) (width 0.25) (layer F.Cu) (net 17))
 (segment (start 57.15 122.301) (end 59.436 120.015) (width 0.25) (layer F.Cu) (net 17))
 (segment (start 54.483 125.349) (end 56.007 125.349) (width 0.25) (layer F.Cu) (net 17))
 (segment (start 56.007 125.349) (end 57.15 124.206) (width 0.25) (layer F.Cu) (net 17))
 (segment (start 57.15 124.206) (end 57.15 122.301) (width 0.25) (layer F.Cu) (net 17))
 (segment (start 59.6646 117.8814) (end 59.6646 115.4684) (width 0.25) (layer F.Cu) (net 18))
 (segment (start 54.483 122.809) (end 54.483 121.6954) (width 0.25) (layer F.Cu) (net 18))
 (segment (start 54.483 121.6954) (end 54.8934 121.285) (width 0.25) (layer F.Cu) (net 18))
 (segment (start 56.261 121.285) (end 59.6646 117.8814) (width 0.25) (layer F.Cu) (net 18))
 (segment (start 54.8934 121.285) (end 56.261 121.285) (width 0.25) (layer F.Cu) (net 18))
 (segment (start 47.625 106.045) (end 47.625 121.031) (width 0.25) (layer F.Cu) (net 23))
 (segment (start 47.625 121.031) (end 49.403 122.809) (width 0.25) (layer F.Cu) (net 23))
 (segment (start 50.292 103.378) (end 47.625 106.045) (width 0.25) (layer F.Cu) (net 23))
 (segment (start 52.0954 97.947944) (end 53.467 96.576344) (width 0.25) (layer B.Cu) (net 24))
 (segment (start 52.0954 99.9236) (end 52.0954 97.947944) (width 0.25) (layer B.Cu) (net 24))
 (segment (start 53.467 96.576344) (end 53.467 96.52) (width 0.25) (layer B.Cu) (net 24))
 (segment (start 54.8005 96.52) (end 56.0705 95.25) (width 0.25) (layer B.Cu) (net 24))
 (segment (start 53.467 96.52) (end 54.8005 96.52) (width 0.25) (layer B.Cu) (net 24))
 (segment (start 43.7515 95.3135) (end 43.2435 95.3135) (width 0.25) (layer B.Cu) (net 25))
 (segment (start 45.72 93.345) (end 43.7515 95.3135) (width 0.25) (layer B.Cu) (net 25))
 (segment (start 47.625 95.25) (end 48.4505 95.25) (width 0.25) (layer B.Cu) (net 25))
 (segment (start 45.72 93.345) (end 47.625 95.25) (width 0.25) (layer B.Cu) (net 25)))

